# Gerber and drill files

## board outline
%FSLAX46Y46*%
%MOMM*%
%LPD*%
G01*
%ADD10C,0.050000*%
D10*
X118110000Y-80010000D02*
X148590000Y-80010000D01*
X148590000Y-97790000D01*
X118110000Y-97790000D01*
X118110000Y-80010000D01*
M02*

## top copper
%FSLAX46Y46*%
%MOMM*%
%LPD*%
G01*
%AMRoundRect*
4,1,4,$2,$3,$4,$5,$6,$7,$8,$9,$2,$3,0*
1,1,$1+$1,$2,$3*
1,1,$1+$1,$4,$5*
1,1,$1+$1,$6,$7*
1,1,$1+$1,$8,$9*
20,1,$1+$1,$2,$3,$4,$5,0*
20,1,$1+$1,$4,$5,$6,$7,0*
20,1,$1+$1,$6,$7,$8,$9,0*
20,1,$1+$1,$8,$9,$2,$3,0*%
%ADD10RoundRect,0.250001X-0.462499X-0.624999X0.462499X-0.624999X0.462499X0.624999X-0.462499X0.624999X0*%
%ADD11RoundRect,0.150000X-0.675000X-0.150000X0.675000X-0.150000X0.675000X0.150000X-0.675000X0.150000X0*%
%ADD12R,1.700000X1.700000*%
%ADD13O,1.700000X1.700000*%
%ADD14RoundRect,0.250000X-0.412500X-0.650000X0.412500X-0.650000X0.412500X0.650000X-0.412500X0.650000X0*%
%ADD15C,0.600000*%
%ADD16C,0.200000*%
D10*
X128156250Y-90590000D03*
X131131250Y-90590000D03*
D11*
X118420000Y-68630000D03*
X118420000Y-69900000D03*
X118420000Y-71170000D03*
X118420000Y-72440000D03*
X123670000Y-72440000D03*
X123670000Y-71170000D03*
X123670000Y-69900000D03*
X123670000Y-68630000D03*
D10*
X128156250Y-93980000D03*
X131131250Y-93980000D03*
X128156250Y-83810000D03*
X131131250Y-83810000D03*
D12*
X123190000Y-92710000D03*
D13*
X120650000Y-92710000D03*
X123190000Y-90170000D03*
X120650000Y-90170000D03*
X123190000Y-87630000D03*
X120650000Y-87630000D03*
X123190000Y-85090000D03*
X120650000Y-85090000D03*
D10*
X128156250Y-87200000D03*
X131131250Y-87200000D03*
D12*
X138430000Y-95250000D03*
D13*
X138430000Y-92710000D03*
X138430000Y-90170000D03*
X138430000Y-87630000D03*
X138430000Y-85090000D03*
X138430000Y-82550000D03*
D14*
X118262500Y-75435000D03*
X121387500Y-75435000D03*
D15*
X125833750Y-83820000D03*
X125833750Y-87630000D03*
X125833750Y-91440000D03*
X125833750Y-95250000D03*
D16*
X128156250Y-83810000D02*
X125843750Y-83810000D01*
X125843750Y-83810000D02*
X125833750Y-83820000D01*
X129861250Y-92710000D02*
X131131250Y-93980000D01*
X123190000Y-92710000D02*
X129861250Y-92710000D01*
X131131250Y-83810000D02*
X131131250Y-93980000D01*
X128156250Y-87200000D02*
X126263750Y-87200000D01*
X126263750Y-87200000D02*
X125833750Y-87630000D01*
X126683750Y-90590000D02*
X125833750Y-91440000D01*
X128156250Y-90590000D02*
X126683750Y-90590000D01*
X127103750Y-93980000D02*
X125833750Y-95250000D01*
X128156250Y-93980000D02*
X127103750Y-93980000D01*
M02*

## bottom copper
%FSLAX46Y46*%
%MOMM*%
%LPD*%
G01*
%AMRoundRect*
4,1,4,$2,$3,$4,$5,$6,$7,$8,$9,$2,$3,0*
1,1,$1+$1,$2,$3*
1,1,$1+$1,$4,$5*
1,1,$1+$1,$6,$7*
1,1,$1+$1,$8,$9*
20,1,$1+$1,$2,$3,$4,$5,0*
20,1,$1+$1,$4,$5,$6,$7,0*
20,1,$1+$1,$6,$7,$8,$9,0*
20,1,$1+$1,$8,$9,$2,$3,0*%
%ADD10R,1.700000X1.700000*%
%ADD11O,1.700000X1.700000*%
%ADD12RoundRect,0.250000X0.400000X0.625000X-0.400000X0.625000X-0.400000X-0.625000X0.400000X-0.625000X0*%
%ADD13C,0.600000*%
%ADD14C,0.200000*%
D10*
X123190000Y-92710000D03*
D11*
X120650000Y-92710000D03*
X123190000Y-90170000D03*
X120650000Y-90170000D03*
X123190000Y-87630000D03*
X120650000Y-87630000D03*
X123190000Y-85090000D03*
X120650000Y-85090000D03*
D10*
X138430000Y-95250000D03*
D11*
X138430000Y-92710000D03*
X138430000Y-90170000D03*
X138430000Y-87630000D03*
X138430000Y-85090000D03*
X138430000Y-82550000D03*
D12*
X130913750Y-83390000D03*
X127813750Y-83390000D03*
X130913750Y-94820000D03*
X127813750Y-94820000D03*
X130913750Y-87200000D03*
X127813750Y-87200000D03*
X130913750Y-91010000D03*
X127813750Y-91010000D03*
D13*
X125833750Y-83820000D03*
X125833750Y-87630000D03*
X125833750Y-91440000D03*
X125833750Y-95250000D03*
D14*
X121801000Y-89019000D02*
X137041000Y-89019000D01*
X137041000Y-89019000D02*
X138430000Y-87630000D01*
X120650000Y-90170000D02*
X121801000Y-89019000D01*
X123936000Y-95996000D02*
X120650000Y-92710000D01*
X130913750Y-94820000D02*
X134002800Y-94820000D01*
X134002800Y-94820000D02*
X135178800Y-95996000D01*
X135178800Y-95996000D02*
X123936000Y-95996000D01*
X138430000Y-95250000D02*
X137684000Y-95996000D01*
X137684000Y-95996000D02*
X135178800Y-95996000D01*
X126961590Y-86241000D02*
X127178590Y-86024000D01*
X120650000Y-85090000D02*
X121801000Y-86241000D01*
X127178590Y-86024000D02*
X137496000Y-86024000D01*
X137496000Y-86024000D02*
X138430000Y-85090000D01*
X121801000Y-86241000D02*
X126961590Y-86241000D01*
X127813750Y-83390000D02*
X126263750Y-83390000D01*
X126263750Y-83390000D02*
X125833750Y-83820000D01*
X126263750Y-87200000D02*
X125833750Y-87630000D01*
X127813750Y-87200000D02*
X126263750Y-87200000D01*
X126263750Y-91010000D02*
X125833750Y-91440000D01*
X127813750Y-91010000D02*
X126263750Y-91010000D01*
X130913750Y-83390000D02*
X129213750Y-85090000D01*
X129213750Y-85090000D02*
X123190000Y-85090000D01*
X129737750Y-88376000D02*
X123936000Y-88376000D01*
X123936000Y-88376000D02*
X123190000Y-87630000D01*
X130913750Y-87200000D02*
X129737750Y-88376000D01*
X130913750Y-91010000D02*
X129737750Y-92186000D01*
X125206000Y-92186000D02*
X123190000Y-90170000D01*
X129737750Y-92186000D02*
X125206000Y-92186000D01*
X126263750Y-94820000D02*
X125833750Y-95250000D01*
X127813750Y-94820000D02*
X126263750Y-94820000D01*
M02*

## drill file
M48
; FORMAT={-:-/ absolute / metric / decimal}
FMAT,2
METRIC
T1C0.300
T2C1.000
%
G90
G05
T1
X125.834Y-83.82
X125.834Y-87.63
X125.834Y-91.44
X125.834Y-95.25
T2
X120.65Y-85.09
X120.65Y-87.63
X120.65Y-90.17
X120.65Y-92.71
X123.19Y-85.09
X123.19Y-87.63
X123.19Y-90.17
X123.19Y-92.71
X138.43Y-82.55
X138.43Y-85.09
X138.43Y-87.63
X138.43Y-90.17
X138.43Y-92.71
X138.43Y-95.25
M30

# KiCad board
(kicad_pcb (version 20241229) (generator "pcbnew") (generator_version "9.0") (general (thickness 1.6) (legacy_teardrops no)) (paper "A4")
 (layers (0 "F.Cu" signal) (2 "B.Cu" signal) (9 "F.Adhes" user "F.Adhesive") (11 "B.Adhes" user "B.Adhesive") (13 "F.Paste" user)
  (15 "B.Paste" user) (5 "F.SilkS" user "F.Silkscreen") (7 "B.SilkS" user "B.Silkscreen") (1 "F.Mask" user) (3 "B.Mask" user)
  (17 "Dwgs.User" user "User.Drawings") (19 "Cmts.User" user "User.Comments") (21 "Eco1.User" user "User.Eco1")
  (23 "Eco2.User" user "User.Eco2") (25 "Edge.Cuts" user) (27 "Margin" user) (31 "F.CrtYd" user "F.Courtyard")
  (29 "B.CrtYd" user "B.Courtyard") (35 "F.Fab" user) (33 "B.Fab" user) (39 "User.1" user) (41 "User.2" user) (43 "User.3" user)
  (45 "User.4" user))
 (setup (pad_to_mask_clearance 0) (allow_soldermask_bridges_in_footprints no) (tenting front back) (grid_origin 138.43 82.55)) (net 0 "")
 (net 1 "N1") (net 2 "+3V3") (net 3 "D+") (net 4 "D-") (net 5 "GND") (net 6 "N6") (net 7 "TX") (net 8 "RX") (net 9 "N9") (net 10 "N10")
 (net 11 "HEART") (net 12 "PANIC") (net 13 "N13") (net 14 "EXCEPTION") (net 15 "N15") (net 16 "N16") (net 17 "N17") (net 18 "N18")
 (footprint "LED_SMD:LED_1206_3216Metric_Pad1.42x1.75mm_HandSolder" (layer "F.Cu") (at 129.64375 90.59)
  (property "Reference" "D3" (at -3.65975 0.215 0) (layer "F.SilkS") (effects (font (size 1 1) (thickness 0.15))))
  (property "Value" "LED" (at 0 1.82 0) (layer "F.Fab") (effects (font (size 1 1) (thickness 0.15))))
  (pad "1" smd roundrect (at -1.4875 0) (size 1.425 1.75) (layers "F.Cu" "F.Mask" "F.Paste") (roundrect_rratio 0.175439) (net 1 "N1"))
  (pad "2" smd roundrect (at 1.4875 0) (size 1.425 1.75) (layers "F.Cu" "F.Mask" "F.Paste") (roundrect_rratio 0.175439) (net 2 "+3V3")))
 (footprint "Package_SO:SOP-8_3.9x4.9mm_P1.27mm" (layer "F.Cu") (at 121.045 70.535)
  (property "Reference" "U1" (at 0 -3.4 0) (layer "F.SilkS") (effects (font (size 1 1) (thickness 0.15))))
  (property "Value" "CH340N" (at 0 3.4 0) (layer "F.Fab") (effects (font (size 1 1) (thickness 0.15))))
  (pad "1" smd roundrect (at -2.625 -1.905) (size 1.65 0.6) (layers "F.Cu" "F.Mask" "F.Paste") (roundrect_rratio 0.25) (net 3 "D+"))
  (pad "2" smd roundrect (at -2.625 -0.635) (size 1.65 0.6) (layers "F.Cu" "F.Mask" "F.Paste") (roundrect_rratio 0.25) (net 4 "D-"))
  (pad "3" smd roundrect (at -2.625 0.635) (size 1.65 0.6) (layers "F.Cu" "F.Mask" "F.Paste") (roundrect_rratio 0.25) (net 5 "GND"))
  (pad "4" smd roundrect (at -2.625 1.905) (size 1.65 0.6) (layers "F.Cu" "F.Mask" "F.Paste") (roundrect_rratio 0.25) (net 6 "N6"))
  (pad "5" smd roundrect (at 2.625 1.905) (size 1.65 0.6) (layers "F.Cu" "F.Mask" "F.Paste") (roundrect_rratio 0.25) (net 2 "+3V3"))
  (pad "6" smd roundrect (at 2.625 0.635) (size 1.65 0.6) (layers "F.Cu" "F.Mask" "F.Paste") (roundrect_rratio 0.25) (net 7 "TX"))
  (pad "7" smd roundrect (at 2.625 -0.635) (size 1.65 0.6) (layers "F.Cu" "F.Mask" "F.Paste") (roundrect_rratio 0.25) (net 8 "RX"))
  (pad "8" smd roundrect (at 2.625 -1.905) (size 1.65 0.6) (layers "F.Cu" "F.Mask" "F.Paste") (roundrect_rratio 0.25) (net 2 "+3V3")))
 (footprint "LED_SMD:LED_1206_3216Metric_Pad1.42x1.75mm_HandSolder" (layer "F.Cu") (at 129.64375 93.98)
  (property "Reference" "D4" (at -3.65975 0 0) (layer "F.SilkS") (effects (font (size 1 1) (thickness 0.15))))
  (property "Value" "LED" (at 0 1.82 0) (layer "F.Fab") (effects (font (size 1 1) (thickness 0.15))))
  (pad "1" smd roundrect (at -1.4875 0) (size 1.425 1.75) (layers "F.Cu" "F.Mask" "F.Paste") (roundrect_rratio 0.175439) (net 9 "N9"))
  (pad "2" smd roundrect (at 1.4875 0) (size 1.425 1.75) (layers "F.Cu" "F.Mask" "F.Paste") (roundrect_rratio 0.175439) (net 2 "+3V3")))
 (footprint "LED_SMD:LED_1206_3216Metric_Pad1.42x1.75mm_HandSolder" (layer "F.Cu") (at 129.64375 83.81)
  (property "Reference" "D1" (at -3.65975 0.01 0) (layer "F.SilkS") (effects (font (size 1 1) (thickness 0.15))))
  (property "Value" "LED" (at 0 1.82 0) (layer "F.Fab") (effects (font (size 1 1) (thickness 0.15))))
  (pad "1" smd roundrect (at -1.4875 0) (size 1.425 1.75) (layers "F.Cu" "F.Mask" "F.Paste") (roundrect_rratio 0.175439) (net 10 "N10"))
  (pad "2" smd roundrect (at 1.4875 0) (size 1.425 1.75) (layers "F.Cu" "F.Mask" "F.Paste") (roundrect_rratio 0.175439) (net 2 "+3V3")))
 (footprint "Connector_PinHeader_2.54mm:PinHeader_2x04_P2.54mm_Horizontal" (layer "F.Cu") (at 123.19 92.71 180)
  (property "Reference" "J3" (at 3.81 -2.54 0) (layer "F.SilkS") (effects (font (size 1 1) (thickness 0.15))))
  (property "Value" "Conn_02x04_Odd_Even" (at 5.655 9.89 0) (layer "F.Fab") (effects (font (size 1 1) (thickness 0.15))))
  (pad "1" thru_hole rect (at 0 0 180) (size 1.7 1.7) (drill 1) (layers "*.Cu" "*.Mask") (remove_unused_layers no) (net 2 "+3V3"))
  (pad "2" thru_hole oval (at 2.54 0 180) (size 1.7 1.7) (drill 1) (layers "*.Cu" "*.Mask") (remove_unused_layers no) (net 5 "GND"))
  (pad "3" thru_hole oval (at 0 2.54 180) (size 1.7 1.7) (drill 1) (layers "*.Cu" "*.Mask") (remove_unused_layers no) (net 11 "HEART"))
  (pad "4" thru_hole oval (at 2.54 2.54 180) (size 1.7 1.7) (drill 1) (layers "*.Cu" "*.Mask") (remove_unused_layers no) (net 7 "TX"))
  (pad "5" thru_hole oval (at 0 5.08 180) (size 1.7 1.7) (drill 1) (layers "*.Cu" "*.Mask") (remove_unused_layers no) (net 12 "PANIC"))
  (pad "6" thru_hole oval (at 2.54 5.08 180) (size 1.7 1.7) (drill 1) (layers "*.Cu" "*.Mask") (remove_unused_layers no) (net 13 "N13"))
  (pad "7" thru_hole oval (at 0 7.62 180) (size 1.7 1.7) (drill 1) (layers "*.Cu" "*.Mask") (remove_unused_layers no) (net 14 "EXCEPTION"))
  (pad "8" thru_hole oval (at 2.54 7.62 180) (size 1.7 1.7) (drill 1) (layers "*.Cu" "*.Mask") (remove_unused_layers no) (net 8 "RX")))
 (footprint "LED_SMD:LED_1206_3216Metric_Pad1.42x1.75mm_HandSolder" (layer "F.Cu") (at 129.64375 87.2)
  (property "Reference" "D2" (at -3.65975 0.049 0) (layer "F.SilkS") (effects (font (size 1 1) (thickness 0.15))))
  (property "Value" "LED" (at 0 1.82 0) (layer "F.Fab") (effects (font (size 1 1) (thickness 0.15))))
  (pad "1" smd roundrect (at -1.4875 0) (size 1.425 1.75) (layers "F.Cu" "F.Mask" "F.Paste") (roundrect_rratio 0.175439) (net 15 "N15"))
  (pad "2" smd roundrect (at 1.4875 0) (size 1.425 1.75) (layers "F.Cu" "F.Mask" "F.Paste") (roundrect_rratio 0.175439) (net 2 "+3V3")))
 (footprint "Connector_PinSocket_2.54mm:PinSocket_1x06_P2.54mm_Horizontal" (layer "F.Cu") (at 138.43 95.25 180)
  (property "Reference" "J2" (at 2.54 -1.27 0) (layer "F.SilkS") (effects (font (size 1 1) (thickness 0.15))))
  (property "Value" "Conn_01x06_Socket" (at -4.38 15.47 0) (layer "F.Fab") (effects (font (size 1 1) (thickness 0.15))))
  (pad "1" thru_hole rect (at 0 0 180) (size 1.7 1.7) (drill 1) (layers "*.Cu" "*.Mask") (remove_unused_layers no) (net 5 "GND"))
  (pad "2" thru_hole oval (at 0 2.54 180) (size 1.7 1.7) (drill 1) (layers "*.Cu" "*.Mask") (remove_unused_layers no) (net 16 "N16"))
  (pad "3" thru_hole oval (at 0 5.08 180) (size 1.7 1.7) (drill 1) (layers "*.Cu" "*.Mask") (remove_unused_layers no) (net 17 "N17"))
  (pad "4" thru_hole oval (at 0 7.62 180) (size 1.7 1.7) (drill 1) (layers "*.Cu" "*.Mask") (remove_unused_layers no) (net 7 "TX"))
  (pad "5" thru_hole oval (at 0 10.16 180) (size 1.7 1.7) (drill 1) (layers "*.Cu" "*.Mask") (remove_unused_layers no) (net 8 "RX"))
  (pad "6" thru_hole oval (at 0 12.7 180) (size 1.7 1.7) (drill 1) (layers "*.Cu" "*.Mask") (remove_unused_layers no) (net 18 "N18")))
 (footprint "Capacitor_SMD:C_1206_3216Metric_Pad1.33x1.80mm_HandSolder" (layer "F.Cu") (at 119.825 75.435)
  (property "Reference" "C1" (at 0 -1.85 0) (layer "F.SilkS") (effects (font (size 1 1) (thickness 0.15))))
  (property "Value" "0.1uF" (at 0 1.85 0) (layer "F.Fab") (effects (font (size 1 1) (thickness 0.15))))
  (pad "1" smd roundrect (at -1.5625 0) (size 1.325 1.8) (layers "F.Cu" "F.Mask" "F.Paste") (roundrect_rratio 0.188679) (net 2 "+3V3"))
  (pad "2" smd roundrect (at 1.5625 0) (size 1.325 1.8) (layers "F.Cu" "F.Mask" "F.Paste") (roundrect_rratio 0.188679) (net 5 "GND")))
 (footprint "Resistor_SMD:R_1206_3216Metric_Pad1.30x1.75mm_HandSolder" (layer "B.Cu") (at 129.36375 83.39 180)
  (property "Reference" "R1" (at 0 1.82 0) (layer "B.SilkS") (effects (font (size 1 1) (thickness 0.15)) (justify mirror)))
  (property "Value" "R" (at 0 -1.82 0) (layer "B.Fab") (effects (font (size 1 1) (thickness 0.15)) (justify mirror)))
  (pad "1" smd roundrect (at -1.55 0 180) (size 1.3 1.75) (layers "B.Cu" "B.Mask" "B.Paste") (roundrect_rratio 0.192308)
   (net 14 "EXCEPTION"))
  (pad "2" smd roundrect (at 1.55 0 180) (size 1.3 1.75) (layers "B.Cu" "B.Mask" "B.Paste") (roundrect_rratio 0.192308) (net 10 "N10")))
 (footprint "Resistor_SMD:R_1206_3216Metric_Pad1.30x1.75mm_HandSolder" (layer "B.Cu") (at 129.36375 94.82 180)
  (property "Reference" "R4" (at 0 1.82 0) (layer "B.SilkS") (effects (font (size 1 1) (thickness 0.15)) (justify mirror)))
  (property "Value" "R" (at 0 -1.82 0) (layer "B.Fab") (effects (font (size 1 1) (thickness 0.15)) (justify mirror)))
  (pad "1" smd roundrect (at -1.55 0 180) (size 1.3 1.75) (layers "B.Cu" "B.Mask" "B.Paste") (roundrect_rratio 0.192308) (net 5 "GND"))
  (pad "2" smd roundrect (at 1.55 0 180) (size 1.3 1.75) (layers "B.Cu" "B.Mask" "B.Paste") (roundrect_rratio 0.192308) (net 9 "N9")))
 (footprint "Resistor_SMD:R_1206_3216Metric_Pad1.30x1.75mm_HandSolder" (layer "B.Cu") (at 129.36375 87.2 180)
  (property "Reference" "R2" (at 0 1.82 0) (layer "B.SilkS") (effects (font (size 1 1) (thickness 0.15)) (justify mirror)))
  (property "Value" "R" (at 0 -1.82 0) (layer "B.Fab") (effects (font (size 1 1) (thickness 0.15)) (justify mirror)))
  (pad "1" smd roundrect (at -1.55 0 180) (size 1.3 1.75) (layers "B.Cu" "B.Mask" "B.Paste") (roundrect_rratio 0.192308) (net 12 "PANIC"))
  (pad "2" smd roundrect (at 1.55 0 180) (size 1.3 1.75) (layers "B.Cu" "B.Mask" "B.Paste") (roundrect_rratio 0.192308) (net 15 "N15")))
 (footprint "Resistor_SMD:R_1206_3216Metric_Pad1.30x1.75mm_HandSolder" (layer "B.Cu") (at 129.36375 91.01 180)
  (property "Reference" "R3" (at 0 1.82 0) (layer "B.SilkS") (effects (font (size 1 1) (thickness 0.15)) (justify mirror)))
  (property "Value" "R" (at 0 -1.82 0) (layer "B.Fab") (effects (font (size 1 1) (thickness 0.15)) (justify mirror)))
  (pad "1" smd roundrect (at -1.55 0 180) (size 1.3 1.75) (layers "B.Cu" "B.Mask" "B.Paste") (roundrect_rratio 0.192308) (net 11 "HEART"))
  (pad "2" smd roundrect (at 1.55 0 180) (size 1.3 1.75) (layers "B.Cu" "B.Mask" "B.Paste") (roundrect_rratio 0.192308) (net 1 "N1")))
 (gr_rect (start 118.11 80.01) (end 148.59 97.79) (stroke (width 0.05) (type default)) (fill no) (layer "Edge.Cuts"))
 (segment (start 121.801 89.019) (end 137.041 89.019) (width 0.2) (layer "B.Cu") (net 7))
 (segment (start 137.041 89.019) (end 138.43 87.63) (width 0.2) (layer "B.Cu") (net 7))
 (segment (start 120.65 90.17) (end 121.801 89.019) (width 0.2) (layer "B.Cu") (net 7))
 (segment (start 123.936 95.996) (end 120.65 92.71) (width 0.2) (layer "B.Cu") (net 5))
 (segment (start 130.91375 94.82) (end 134.0028 94.82) (width 0.2) (layer "B.Cu") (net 5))
 (segment (start 134.0028 94.82) (end 135.1788 95.996) (width 0.2) (layer "B.Cu") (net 5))
 (segment (start 135.1788 95.996) (end 123.936 95.996) (width 0.2) (layer "B.Cu") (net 5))
 (segment (start 138.43 95.25) (end 137.684 95.996) (width 0.2) (layer "B.Cu") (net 5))
 (segment (start 137.684 95.996) (end 135.1788 95.996) (width 0.2) (layer "B.Cu") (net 5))
 (segment (start 126.96159 86.241) (end 127.17859 86.024) (width 0.2) (layer "B.Cu") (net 8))
 (segment (start 120.65 85.09) (end 121.801 86.241) (width 0.2) (layer "B.Cu") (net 8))
 (segment (start 127.17859 86.024) (end 137.496 86.024) (width 0.2) (layer "B.Cu") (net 8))
 (segment (start 137.496 86.024) (end 138.43 85.09) (width 0.2) (layer "B.Cu") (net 8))
 (segment (start 121.801 86.241) (end 126.96159 86.241) (width 0.2) (layer "B.Cu") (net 8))
 (segment (start 128.15625 83.81) (end 125.84375 83.81) (width 0.2) (layer "F.Cu") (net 10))
 (segment (start 125.84375 83.81) (end 125.83375 83.82) (width 0.2) (layer "F.Cu") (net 10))
 (via (at 125.83375 83.82) (size 0.6) (drill 0.3) (layers "F.Cu" "B.Cu") (free yes) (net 10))
 (segment (start 127.81375 83.39) (end 126.26375 83.39) (width 0.2) (layer "B.Cu") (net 10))
 (segment (start 126.26375 83.39) (end 125.83375 83.82) (width 0.2) (layer "B.Cu") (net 10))
 (segment (start 129.86125 92.71) (end 131.13125 93.98) (width 0.2) (layer "F.Cu") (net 2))
 (segment (start 123.19 92.71) (end 129.86125 92.71) (width 0.2) (layer "F.Cu") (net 2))
 (segment (start 131.13125 83.81) (end 131.13125 93.98) (width 0.2) (layer "F.Cu") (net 2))
 (segment (start 128.15625 87.2) (end 126.26375 87.2) (width 0.2) (layer "F.Cu") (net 15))
 (segment (start 126.26375 87.2) (end 125.83375 87.63) (width 0.2) (layer "F.Cu") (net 15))
 (via (at 125.83375 87.63) (size 0.6) (drill 0.3) (layers "F.Cu" "B.Cu") (free yes) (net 15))
 (segment (start 126.26375 87.2) (end 125.83375 87.63) (width 0.2) (layer "B.Cu") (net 15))
 (segment (start 127.81375 87.2) (end 126.26375 87.2) (width 0.2) (layer "B.Cu") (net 15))
 (segment (start 126.68375 90.59) (end 125.83375 91.44) (width 0.2) (layer "F.Cu") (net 1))
 (segment (start 128.15625 90.59) (end 126.68375 90.59) (width 0.2) (layer "F.Cu") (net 1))
 (via (at 125.83375 91.44) (size 0.6) (drill 0.3) (layers "F.Cu" "B.Cu") (free yes) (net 1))
 (segment (start 126.26375 91.01) (end 125.83375 91.44) (width 0.2) (layer "B.Cu") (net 1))
 (segment (start 127.81375 91.01) (end 126.26375 91.01) (width 0.2) (layer "B.Cu") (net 1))
 (segment (start 130.91375 83.39) (end 129.21375 85.09) (width 0.2) (layer "B.Cu") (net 14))
 (segment (start 129.21375 85.09) (end 123.19 85.09) (width 0.2) (layer "B.Cu") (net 14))
 (segment (start 129.73775 88.376) (end 123.936 88.376) (width 0.2) (layer "B.Cu") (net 12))
 (segment (start 123.936 88.376) (end 123.19 87.63) (width 0.2) (layer "B.Cu") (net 12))
 (segment (start 130.91375 87.2) (end 129.73775 88.376) (width 0.2) (layer "B.Cu") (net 12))
 (segment (start 130.91375 91.01) (end 129.73775 92.186) (width 0.2) (layer "B.Cu") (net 11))
 (segment (start 125.206 92.186) (end 123.19 90.17) (width 0.2) (layer "B.Cu") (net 11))
 (segment (start 129.73775 92.186) (end 125.206 92.186) (width 0.2) (layer "B.Cu") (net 11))
 (segment (start 127.10375 93.98) (end 125.83375 95.25) (width 0.2) (layer "F.Cu") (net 9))
 (segment (start 128.15625 93.98) (end 127.10375 93.98) (width 0.2) (layer "F.Cu") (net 9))
 (via (at 125.83375 95.25) (size 0.6) (drill 0.3) (layers "F.Cu" "B.Cu") (free yes) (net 9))
 (segment (start 126.26375 94.82) (end 125.83375 95.25) (width 0.2) (layer "B.Cu") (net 9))
 (segment (start 127.81375 94.82) (end 126.26375 94.82) (width 0.2) (layer "B.Cu") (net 9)))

